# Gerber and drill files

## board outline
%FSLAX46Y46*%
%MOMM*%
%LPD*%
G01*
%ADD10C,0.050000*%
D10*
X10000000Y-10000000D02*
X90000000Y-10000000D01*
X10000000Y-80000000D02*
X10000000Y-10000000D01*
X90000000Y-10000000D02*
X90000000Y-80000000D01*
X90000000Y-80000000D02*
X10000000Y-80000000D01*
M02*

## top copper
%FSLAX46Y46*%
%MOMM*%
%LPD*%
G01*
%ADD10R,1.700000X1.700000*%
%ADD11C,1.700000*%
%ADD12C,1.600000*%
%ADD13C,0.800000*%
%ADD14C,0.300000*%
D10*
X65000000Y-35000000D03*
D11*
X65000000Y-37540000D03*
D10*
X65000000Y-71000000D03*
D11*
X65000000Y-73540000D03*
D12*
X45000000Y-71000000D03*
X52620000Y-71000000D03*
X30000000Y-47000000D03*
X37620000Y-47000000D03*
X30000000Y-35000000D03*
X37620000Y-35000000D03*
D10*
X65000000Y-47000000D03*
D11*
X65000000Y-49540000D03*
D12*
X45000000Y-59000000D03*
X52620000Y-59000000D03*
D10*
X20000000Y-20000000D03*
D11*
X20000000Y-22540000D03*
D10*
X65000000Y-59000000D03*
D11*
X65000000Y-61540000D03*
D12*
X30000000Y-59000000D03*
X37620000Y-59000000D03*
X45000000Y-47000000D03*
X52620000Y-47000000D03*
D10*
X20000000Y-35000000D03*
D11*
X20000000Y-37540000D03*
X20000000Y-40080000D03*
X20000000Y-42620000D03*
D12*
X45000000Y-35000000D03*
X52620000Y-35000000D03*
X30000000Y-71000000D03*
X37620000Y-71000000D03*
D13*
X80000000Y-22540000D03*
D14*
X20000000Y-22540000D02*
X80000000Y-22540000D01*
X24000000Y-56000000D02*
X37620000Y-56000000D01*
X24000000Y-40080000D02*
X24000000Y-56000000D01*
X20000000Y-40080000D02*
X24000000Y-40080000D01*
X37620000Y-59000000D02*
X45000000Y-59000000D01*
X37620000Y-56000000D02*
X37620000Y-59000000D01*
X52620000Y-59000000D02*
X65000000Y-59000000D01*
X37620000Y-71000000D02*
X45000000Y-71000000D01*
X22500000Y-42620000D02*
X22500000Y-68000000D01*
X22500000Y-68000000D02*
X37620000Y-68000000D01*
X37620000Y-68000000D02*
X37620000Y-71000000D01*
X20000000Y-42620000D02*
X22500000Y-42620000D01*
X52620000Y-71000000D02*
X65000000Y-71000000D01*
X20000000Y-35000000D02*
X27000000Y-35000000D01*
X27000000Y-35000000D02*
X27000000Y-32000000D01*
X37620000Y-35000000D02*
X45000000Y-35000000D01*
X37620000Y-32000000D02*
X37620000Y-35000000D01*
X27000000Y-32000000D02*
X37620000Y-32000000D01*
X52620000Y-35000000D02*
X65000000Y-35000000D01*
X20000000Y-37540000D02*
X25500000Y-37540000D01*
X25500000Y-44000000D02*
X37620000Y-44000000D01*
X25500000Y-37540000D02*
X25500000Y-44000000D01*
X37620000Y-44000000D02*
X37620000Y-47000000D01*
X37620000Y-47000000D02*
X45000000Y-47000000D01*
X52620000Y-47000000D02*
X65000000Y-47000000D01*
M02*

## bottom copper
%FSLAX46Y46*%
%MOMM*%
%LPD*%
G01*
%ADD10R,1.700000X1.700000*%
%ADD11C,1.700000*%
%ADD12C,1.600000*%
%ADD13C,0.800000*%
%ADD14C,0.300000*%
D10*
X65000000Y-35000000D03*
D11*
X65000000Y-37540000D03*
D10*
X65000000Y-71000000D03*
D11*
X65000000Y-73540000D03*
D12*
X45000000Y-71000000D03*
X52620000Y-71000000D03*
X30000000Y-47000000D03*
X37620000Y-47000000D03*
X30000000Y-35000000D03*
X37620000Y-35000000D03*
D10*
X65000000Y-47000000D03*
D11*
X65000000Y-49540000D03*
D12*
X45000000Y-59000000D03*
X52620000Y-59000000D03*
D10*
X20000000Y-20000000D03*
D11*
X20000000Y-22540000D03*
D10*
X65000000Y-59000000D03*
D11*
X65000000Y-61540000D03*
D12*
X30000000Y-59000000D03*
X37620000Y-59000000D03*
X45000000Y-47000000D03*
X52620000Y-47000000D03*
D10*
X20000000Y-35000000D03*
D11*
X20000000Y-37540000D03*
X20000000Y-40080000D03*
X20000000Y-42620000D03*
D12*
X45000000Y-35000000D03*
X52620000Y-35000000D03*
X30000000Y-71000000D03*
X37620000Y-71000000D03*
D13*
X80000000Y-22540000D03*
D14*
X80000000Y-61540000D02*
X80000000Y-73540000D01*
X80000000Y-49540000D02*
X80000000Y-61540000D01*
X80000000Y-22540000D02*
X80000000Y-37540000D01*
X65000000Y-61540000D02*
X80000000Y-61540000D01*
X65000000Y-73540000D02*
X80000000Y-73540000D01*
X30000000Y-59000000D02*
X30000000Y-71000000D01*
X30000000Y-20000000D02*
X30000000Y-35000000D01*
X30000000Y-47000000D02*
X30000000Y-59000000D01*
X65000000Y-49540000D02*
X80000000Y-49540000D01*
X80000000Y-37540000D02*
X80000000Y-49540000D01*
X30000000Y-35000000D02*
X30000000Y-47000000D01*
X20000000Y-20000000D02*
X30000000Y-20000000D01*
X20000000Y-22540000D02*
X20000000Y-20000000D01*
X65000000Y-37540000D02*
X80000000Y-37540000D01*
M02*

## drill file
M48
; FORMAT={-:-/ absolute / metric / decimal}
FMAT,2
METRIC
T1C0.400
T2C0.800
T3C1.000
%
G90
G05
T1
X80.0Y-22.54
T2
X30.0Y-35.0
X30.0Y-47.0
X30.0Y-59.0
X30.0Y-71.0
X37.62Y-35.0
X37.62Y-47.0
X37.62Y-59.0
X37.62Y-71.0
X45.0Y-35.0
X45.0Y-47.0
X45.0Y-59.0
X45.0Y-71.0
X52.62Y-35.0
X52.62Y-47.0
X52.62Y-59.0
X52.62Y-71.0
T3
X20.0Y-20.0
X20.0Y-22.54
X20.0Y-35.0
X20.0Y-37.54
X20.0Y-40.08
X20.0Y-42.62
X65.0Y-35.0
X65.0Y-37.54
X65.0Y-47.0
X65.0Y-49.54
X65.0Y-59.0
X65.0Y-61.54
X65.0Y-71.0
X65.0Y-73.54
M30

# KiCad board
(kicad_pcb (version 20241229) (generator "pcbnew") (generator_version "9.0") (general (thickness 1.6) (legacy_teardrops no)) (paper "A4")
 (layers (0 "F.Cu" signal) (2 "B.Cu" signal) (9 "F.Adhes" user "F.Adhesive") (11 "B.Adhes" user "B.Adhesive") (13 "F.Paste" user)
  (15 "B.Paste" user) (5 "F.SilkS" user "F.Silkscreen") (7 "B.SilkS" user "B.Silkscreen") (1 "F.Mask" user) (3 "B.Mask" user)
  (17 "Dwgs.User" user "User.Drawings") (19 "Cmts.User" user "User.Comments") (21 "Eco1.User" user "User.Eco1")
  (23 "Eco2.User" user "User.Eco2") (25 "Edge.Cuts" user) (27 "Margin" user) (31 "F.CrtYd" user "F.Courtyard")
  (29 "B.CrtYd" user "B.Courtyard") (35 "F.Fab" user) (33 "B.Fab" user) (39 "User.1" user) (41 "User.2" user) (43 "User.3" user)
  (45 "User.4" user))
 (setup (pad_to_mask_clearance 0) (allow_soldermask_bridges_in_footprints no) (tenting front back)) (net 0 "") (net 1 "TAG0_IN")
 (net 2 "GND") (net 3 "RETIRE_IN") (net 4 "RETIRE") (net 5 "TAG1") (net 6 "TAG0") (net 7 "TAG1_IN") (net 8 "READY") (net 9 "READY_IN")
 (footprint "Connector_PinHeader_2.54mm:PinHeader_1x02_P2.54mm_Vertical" (layer "F.Cu") (at 65 35)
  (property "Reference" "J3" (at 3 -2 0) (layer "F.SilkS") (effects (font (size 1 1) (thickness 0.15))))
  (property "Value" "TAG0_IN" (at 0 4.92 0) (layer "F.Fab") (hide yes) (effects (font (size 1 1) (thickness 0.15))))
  (pad "1" thru_hole rect (at 0 0) (size 1.7 1.7) (drill 1) (layers "*.Cu" "*.Mask") (remove_unused_layers no) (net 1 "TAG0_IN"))
  (pad "2" thru_hole circle (at 0 2.54) (size 1.7 1.7) (drill 1) (layers "*.Cu" "*.Mask") (remove_unused_layers no) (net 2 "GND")))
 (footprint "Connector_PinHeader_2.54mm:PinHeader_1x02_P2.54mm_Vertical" (layer "F.Cu") (at 65 71)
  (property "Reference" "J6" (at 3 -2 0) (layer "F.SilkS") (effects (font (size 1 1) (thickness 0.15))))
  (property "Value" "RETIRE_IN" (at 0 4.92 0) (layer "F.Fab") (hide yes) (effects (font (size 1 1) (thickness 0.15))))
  (pad "1" thru_hole rect (at 0 0) (size 1.7 1.7) (drill 1) (layers "*.Cu" "*.Mask") (remove_unused_layers no) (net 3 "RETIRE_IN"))
  (pad "2" thru_hole circle (at 0 2.54) (size 1.7 1.7) (drill 1) (layers "*.Cu" "*.Mask") (remove_unused_layers no) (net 2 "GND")))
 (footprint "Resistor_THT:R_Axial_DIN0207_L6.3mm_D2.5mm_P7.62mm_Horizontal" (layer "F.Cu") (at 45 71)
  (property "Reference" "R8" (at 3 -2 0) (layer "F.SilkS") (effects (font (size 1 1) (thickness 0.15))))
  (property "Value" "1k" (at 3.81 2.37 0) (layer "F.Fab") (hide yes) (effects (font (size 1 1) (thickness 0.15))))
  (pad "1" thru_hole circle (at 0 0) (size 1.6 1.6) (drill 0.8) (layers "*.Cu" "*.Mask") (remove_unused_layers no) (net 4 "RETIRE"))
  (pad "2" thru_hole circle (at 7.62 0) (size 1.6 1.6) (drill 0.8) (layers "*.Cu" "*.Mask") (remove_unused_layers no) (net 3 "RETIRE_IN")))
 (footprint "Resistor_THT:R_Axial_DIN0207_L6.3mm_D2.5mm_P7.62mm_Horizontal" (layer "F.Cu") (at 30 47)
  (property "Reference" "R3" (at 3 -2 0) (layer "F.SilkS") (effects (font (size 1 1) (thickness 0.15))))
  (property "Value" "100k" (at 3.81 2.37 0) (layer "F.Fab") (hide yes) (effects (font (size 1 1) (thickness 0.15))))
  (pad "1" thru_hole circle (at 0 0) (size 1.6 1.6) (drill 0.8) (layers "*.Cu" "*.Mask") (remove_unused_layers no) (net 2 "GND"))
  (pad "2" thru_hole circle (at 7.62 0) (size 1.6 1.6) (drill 0.8) (layers "*.Cu" "*.Mask") (remove_unused_layers no) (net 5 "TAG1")))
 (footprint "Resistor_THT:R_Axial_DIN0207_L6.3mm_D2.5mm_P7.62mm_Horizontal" (layer "F.Cu") (at 30 35)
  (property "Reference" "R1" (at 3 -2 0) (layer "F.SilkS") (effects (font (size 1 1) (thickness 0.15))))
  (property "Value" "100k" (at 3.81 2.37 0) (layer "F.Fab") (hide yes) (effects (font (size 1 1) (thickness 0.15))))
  (pad "1" thru_hole circle (at 0 0) (size 1.6 1.6) (drill 0.8) (layers "*.Cu" "*.Mask") (remove_unused_layers no) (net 2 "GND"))
  (pad "2" thru_hole circle (at 7.62 0) (size 1.6 1.6) (drill 0.8) (layers "*.Cu" "*.Mask") (remove_unused_layers no) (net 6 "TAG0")))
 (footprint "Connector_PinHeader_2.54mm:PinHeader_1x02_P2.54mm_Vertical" (layer "F.Cu") (at 65 47)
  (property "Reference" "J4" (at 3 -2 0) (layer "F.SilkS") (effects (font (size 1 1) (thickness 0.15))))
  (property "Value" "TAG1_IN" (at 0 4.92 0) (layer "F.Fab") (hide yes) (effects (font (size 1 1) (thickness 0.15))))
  (pad "1" thru_hole rect (at 0 0) (size 1.7 1.7) (drill 1) (layers "*.Cu" "*.Mask") (remove_unused_layers no) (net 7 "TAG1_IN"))
  (pad "2" thru_hole circle (at 0 2.54) (size 1.7 1.7) (drill 1) (layers "*.Cu" "*.Mask") (remove_unused_layers no) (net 2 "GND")))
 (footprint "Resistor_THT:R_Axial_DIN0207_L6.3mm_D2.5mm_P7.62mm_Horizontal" (layer "F.Cu") (at 45 59)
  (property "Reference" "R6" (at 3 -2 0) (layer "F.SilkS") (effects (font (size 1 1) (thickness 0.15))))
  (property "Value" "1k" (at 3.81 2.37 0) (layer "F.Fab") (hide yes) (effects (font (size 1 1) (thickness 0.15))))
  (pad "1" thru_hole circle (at 0 0) (size 1.6 1.6) (drill 0.8) (layers "*.Cu" "*.Mask") (remove_unused_layers no) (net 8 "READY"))
  (pad "2" thru_hole circle (at 7.62 0) (size 1.6 1.6) (drill 0.8) (layers "*.Cu" "*.Mask") (remove_unused_layers no) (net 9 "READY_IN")))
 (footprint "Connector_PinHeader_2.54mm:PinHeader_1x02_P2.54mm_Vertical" (layer "F.Cu") (at 20 20)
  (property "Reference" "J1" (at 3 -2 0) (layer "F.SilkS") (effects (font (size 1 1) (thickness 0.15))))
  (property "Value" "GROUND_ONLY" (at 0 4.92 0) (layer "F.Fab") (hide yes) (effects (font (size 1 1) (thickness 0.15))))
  (pad "1" thru_hole rect (at 0 0) (size 1.7 1.7) (drill 1) (layers "*.Cu" "*.Mask") (remove_unused_layers no) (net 2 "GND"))
  (pad "2" thru_hole circle (at 0 2.54) (size 1.7 1.7) (drill 1) (layers "*.Cu" "*.Mask") (remove_unused_layers no) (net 2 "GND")))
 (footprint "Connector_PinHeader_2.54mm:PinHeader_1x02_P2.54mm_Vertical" (layer "F.Cu") (at 65 59)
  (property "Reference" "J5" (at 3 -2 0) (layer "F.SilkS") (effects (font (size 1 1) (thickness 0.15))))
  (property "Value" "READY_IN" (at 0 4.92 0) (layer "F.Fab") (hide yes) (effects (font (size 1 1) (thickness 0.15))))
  (pad "1" thru_hole rect (at 0 0) (size 1.7 1.7) (drill 1) (layers "*.Cu" "*.Mask") (remove_unused_layers no) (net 9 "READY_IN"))
  (pad "2" thru_hole circle (at 0 2.54) (size 1.7 1.7) (drill 1) (layers "*.Cu" "*.Mask") (remove_unused_layers no) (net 2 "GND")))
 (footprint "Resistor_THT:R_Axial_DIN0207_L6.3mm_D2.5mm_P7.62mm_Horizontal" (layer "F.Cu") (at 30 59)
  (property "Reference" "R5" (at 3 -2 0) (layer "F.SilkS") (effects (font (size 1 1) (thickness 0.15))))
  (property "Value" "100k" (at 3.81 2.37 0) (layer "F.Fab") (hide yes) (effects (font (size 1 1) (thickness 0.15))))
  (pad "1" thru_hole circle (at 0 0) (size 1.6 1.6) (drill 0.8) (layers "*.Cu" "*.Mask") (remove_unused_layers no) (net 2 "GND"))
  (pad "2" thru_hole circle (at 7.62 0) (size 1.6 1.6) (drill 0.8) (layers "*.Cu" "*.Mask") (remove_unused_layers no) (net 8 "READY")))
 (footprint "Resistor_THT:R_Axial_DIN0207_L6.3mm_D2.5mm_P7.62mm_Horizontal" (layer "F.Cu") (at 45 47)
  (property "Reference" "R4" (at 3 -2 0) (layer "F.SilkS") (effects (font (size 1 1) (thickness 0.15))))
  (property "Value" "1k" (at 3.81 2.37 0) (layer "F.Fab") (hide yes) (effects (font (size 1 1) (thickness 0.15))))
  (pad "1" thru_hole circle (at 0 0) (size 1.6 1.6) (drill 0.8) (layers "*.Cu" "*.Mask") (remove_unused_layers no) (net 5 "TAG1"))
  (pad "2" thru_hole circle (at 7.62 0) (size 1.6 1.6) (drill 0.8) (layers "*.Cu" "*.Mask") (remove_unused_layers no) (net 7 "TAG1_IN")))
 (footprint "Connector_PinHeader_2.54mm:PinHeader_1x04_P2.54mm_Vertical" (layer "F.Cu") (at 20 35)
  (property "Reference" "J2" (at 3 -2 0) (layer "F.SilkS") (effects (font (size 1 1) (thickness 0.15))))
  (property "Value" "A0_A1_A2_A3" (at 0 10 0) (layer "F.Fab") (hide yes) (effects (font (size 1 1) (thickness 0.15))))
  (pad "1" thru_hole rect (at 0 0) (size 1.7 1.7) (drill 1) (layers "*.Cu" "*.Mask") (remove_unused_layers no) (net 6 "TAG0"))
  (pad "2" thru_hole circle (at 0 2.54) (size 1.7 1.7) (drill 1) (layers "*.Cu" "*.Mask") (remove_unused_layers no) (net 5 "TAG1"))
  (pad "3" thru_hole circle (at 0 5.08) (size 1.7 1.7) (drill 1) (layers "*.Cu" "*.Mask") (remove_unused_layers no) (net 8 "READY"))
  (pad "4" thru_hole circle (at 0 7.62) (size 1.7 1.7) (drill 1) (layers "*.Cu" "*.Mask") (remove_unused_layers no) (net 4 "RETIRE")))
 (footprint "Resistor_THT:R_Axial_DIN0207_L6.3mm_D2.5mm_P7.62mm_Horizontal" (layer "F.Cu") (at 45 35)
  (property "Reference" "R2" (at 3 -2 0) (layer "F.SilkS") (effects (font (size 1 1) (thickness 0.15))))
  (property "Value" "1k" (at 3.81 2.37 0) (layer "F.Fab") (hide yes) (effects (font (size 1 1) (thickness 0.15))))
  (pad "1" thru_hole circle (at 0 0) (size 1.6 1.6) (drill 0.8) (layers "*.Cu" "*.Mask") (remove_unused_layers no) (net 6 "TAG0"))
  (pad "2" thru_hole circle (at 7.62 0) (size 1.6 1.6) (drill 0.8) (layers "*.Cu" "*.Mask") (remove_unused_layers no) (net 1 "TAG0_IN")))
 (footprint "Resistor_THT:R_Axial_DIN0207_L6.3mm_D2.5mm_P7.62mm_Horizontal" (layer "F.Cu") (at 30 71)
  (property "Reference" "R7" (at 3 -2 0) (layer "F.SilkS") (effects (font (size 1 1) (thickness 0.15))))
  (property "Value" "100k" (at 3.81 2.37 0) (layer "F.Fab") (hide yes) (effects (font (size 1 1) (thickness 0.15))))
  (pad "1" thru_hole circle (at 0 0) (size 1.6 1.6) (drill 0.8) (layers "*.Cu" "*.Mask") (remove_unused_layers no) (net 2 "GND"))
  (pad "2" thru_hole circle (at 7.62 0) (size 1.6 1.6) (drill 0.8) (layers "*.Cu" "*.Mask") (remove_unused_layers no) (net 4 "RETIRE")))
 (gr_line (start 10 10) (end 90 10) (stroke (width 0.05) (type default)) (layer "Edge.Cuts"))
 (gr_line (start 10 80) (end 10 10) (stroke (width 0.05) (type default)) (layer "Edge.Cuts"))
 (gr_line (start 90 10) (end 90 80) (stroke (width 0.05) (type default)) (layer "Edge.Cuts"))
 (gr_line (start 90 80) (end 10 80) (stroke (width 0.05) (type default)) (layer "Edge.Cuts"))
 (segment (start 20 22.54) (end 80 22.54) (width 0.3) (layer "F.Cu") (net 2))
 (via (at 80 22.54) (size 0.8) (drill 0.4) (layers "F.Cu" "B.Cu") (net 2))
 (segment (start 80 61.54) (end 80 73.54) (width 0.3) (layer "B.Cu") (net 2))
 (segment (start 80 49.54) (end 80 61.54) (width 0.3) (layer "B.Cu") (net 2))
 (segment (start 80 22.54) (end 80 37.54) (width 0.3) (layer "B.Cu") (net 2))
 (segment (start 65 61.54) (end 80 61.54) (width 0.3) (layer "B.Cu") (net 2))
 (segment (start 65 73.54) (end 80 73.54) (width 0.3) (layer "B.Cu") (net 2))
 (segment (start 30 59) (end 30 71) (width 0.3) (layer "B.Cu") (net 2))
 (segment (start 30 20) (end 30 35) (width 0.3) (layer "B.Cu") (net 2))
 (segment (start 30 47) (end 30 59) (width 0.3) (layer "B.Cu") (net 2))
 (segment (start 65 49.54) (end 80 49.54) (width 0.3) (layer "B.Cu") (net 2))
 (segment (start 80 37.54) (end 80 49.54) (width 0.3) (layer "B.Cu") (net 2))
 (segment (start 30 35) (end 30 47) (width 0.3) (layer "B.Cu") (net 2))
 (segment (start 20 20) (end 30 20) (width 0.3) (layer "B.Cu") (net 2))
 (segment (start 20 22.54) (end 20 20) (width 0.3) (layer "B.Cu") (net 2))
 (segment (start 65 37.54) (end 80 37.54) (width 0.3) (layer "B.Cu") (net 2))
 (segment (start 24 56) (end 37.62 56) (width 0.3) (layer "F.Cu") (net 8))
 (segment (start 24 40.08) (end 24 56) (width 0.3) (layer "F.Cu") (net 8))
 (segment (start 20 40.08) (end 24 40.08) (width 0.3) (layer "F.Cu") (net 8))
 (segment (start 37.62 59) (end 45 59) (width 0.3) (layer "F.Cu") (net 8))
 (segment (start 37.62 56) (end 37.62 59) (width 0.3) (layer "F.Cu") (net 8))
 (segment (start 52.62 59) (end 65 59) (width 0.3) (layer "F.Cu") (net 9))
 (segment (start 37.62 71) (end 45 71) (width 0.3) (layer "F.Cu") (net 4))
 (segment (start 22.5 42.62) (end 22.5 68) (width 0.3) (layer "F.Cu") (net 4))
 (segment (start 22.5 68) (end 37.62 68) (width 0.3) (layer "F.Cu") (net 4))
 (segment (start 37.62 68) (end 37.62 71) (width 0.3) (layer "F.Cu") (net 4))
 (segment (start 20 42.62) (end 22.5 42.62) (width 0.3) (layer "F.Cu") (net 4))
 (segment (start 52.62 71) (end 65 71) (width 0.3) (layer "F.Cu") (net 3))
 (segment (start 20 35) (end 27 35) (width 0.3) (layer "F.Cu") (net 6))
 (segment (start 27 35) (end 27 32) (width 0.3) (layer "F.Cu") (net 6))
 (segment (start 37.62 35) (end 45 35) (width 0.3) (layer "F.Cu") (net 6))
 (segment (start 37.62 32) (end 37.62 35) (width 0.3) (layer "F.Cu") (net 6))
 (segment (start 27 32) (end 37.62 32) (width 0.3) (layer "F.Cu") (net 6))
 (segment (start 52.62 35) (end 65 35) (width 0.3) (layer "F.Cu") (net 1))
 (segment (start 20 37.54) (end 25.5 37.54) (width 0.3) (layer "F.Cu") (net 5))
 (segment (start 25.5 44) (end 37.62 44) (width 0.3) (layer "F.Cu") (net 5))
 (segment (start 25.5 37.54) (end 25.5 44) (width 0.3) (layer "F.Cu") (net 5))
 (segment (start 37.62 44) (end 37.62 47) (width 0.3) (layer "F.Cu") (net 5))
 (segment (start 37.62 47) (end 45 47) (width 0.3) (layer "F.Cu") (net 5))
 (segment (start 52.62 47) (end 65 47) (width 0.3) (layer "F.Cu") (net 7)))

